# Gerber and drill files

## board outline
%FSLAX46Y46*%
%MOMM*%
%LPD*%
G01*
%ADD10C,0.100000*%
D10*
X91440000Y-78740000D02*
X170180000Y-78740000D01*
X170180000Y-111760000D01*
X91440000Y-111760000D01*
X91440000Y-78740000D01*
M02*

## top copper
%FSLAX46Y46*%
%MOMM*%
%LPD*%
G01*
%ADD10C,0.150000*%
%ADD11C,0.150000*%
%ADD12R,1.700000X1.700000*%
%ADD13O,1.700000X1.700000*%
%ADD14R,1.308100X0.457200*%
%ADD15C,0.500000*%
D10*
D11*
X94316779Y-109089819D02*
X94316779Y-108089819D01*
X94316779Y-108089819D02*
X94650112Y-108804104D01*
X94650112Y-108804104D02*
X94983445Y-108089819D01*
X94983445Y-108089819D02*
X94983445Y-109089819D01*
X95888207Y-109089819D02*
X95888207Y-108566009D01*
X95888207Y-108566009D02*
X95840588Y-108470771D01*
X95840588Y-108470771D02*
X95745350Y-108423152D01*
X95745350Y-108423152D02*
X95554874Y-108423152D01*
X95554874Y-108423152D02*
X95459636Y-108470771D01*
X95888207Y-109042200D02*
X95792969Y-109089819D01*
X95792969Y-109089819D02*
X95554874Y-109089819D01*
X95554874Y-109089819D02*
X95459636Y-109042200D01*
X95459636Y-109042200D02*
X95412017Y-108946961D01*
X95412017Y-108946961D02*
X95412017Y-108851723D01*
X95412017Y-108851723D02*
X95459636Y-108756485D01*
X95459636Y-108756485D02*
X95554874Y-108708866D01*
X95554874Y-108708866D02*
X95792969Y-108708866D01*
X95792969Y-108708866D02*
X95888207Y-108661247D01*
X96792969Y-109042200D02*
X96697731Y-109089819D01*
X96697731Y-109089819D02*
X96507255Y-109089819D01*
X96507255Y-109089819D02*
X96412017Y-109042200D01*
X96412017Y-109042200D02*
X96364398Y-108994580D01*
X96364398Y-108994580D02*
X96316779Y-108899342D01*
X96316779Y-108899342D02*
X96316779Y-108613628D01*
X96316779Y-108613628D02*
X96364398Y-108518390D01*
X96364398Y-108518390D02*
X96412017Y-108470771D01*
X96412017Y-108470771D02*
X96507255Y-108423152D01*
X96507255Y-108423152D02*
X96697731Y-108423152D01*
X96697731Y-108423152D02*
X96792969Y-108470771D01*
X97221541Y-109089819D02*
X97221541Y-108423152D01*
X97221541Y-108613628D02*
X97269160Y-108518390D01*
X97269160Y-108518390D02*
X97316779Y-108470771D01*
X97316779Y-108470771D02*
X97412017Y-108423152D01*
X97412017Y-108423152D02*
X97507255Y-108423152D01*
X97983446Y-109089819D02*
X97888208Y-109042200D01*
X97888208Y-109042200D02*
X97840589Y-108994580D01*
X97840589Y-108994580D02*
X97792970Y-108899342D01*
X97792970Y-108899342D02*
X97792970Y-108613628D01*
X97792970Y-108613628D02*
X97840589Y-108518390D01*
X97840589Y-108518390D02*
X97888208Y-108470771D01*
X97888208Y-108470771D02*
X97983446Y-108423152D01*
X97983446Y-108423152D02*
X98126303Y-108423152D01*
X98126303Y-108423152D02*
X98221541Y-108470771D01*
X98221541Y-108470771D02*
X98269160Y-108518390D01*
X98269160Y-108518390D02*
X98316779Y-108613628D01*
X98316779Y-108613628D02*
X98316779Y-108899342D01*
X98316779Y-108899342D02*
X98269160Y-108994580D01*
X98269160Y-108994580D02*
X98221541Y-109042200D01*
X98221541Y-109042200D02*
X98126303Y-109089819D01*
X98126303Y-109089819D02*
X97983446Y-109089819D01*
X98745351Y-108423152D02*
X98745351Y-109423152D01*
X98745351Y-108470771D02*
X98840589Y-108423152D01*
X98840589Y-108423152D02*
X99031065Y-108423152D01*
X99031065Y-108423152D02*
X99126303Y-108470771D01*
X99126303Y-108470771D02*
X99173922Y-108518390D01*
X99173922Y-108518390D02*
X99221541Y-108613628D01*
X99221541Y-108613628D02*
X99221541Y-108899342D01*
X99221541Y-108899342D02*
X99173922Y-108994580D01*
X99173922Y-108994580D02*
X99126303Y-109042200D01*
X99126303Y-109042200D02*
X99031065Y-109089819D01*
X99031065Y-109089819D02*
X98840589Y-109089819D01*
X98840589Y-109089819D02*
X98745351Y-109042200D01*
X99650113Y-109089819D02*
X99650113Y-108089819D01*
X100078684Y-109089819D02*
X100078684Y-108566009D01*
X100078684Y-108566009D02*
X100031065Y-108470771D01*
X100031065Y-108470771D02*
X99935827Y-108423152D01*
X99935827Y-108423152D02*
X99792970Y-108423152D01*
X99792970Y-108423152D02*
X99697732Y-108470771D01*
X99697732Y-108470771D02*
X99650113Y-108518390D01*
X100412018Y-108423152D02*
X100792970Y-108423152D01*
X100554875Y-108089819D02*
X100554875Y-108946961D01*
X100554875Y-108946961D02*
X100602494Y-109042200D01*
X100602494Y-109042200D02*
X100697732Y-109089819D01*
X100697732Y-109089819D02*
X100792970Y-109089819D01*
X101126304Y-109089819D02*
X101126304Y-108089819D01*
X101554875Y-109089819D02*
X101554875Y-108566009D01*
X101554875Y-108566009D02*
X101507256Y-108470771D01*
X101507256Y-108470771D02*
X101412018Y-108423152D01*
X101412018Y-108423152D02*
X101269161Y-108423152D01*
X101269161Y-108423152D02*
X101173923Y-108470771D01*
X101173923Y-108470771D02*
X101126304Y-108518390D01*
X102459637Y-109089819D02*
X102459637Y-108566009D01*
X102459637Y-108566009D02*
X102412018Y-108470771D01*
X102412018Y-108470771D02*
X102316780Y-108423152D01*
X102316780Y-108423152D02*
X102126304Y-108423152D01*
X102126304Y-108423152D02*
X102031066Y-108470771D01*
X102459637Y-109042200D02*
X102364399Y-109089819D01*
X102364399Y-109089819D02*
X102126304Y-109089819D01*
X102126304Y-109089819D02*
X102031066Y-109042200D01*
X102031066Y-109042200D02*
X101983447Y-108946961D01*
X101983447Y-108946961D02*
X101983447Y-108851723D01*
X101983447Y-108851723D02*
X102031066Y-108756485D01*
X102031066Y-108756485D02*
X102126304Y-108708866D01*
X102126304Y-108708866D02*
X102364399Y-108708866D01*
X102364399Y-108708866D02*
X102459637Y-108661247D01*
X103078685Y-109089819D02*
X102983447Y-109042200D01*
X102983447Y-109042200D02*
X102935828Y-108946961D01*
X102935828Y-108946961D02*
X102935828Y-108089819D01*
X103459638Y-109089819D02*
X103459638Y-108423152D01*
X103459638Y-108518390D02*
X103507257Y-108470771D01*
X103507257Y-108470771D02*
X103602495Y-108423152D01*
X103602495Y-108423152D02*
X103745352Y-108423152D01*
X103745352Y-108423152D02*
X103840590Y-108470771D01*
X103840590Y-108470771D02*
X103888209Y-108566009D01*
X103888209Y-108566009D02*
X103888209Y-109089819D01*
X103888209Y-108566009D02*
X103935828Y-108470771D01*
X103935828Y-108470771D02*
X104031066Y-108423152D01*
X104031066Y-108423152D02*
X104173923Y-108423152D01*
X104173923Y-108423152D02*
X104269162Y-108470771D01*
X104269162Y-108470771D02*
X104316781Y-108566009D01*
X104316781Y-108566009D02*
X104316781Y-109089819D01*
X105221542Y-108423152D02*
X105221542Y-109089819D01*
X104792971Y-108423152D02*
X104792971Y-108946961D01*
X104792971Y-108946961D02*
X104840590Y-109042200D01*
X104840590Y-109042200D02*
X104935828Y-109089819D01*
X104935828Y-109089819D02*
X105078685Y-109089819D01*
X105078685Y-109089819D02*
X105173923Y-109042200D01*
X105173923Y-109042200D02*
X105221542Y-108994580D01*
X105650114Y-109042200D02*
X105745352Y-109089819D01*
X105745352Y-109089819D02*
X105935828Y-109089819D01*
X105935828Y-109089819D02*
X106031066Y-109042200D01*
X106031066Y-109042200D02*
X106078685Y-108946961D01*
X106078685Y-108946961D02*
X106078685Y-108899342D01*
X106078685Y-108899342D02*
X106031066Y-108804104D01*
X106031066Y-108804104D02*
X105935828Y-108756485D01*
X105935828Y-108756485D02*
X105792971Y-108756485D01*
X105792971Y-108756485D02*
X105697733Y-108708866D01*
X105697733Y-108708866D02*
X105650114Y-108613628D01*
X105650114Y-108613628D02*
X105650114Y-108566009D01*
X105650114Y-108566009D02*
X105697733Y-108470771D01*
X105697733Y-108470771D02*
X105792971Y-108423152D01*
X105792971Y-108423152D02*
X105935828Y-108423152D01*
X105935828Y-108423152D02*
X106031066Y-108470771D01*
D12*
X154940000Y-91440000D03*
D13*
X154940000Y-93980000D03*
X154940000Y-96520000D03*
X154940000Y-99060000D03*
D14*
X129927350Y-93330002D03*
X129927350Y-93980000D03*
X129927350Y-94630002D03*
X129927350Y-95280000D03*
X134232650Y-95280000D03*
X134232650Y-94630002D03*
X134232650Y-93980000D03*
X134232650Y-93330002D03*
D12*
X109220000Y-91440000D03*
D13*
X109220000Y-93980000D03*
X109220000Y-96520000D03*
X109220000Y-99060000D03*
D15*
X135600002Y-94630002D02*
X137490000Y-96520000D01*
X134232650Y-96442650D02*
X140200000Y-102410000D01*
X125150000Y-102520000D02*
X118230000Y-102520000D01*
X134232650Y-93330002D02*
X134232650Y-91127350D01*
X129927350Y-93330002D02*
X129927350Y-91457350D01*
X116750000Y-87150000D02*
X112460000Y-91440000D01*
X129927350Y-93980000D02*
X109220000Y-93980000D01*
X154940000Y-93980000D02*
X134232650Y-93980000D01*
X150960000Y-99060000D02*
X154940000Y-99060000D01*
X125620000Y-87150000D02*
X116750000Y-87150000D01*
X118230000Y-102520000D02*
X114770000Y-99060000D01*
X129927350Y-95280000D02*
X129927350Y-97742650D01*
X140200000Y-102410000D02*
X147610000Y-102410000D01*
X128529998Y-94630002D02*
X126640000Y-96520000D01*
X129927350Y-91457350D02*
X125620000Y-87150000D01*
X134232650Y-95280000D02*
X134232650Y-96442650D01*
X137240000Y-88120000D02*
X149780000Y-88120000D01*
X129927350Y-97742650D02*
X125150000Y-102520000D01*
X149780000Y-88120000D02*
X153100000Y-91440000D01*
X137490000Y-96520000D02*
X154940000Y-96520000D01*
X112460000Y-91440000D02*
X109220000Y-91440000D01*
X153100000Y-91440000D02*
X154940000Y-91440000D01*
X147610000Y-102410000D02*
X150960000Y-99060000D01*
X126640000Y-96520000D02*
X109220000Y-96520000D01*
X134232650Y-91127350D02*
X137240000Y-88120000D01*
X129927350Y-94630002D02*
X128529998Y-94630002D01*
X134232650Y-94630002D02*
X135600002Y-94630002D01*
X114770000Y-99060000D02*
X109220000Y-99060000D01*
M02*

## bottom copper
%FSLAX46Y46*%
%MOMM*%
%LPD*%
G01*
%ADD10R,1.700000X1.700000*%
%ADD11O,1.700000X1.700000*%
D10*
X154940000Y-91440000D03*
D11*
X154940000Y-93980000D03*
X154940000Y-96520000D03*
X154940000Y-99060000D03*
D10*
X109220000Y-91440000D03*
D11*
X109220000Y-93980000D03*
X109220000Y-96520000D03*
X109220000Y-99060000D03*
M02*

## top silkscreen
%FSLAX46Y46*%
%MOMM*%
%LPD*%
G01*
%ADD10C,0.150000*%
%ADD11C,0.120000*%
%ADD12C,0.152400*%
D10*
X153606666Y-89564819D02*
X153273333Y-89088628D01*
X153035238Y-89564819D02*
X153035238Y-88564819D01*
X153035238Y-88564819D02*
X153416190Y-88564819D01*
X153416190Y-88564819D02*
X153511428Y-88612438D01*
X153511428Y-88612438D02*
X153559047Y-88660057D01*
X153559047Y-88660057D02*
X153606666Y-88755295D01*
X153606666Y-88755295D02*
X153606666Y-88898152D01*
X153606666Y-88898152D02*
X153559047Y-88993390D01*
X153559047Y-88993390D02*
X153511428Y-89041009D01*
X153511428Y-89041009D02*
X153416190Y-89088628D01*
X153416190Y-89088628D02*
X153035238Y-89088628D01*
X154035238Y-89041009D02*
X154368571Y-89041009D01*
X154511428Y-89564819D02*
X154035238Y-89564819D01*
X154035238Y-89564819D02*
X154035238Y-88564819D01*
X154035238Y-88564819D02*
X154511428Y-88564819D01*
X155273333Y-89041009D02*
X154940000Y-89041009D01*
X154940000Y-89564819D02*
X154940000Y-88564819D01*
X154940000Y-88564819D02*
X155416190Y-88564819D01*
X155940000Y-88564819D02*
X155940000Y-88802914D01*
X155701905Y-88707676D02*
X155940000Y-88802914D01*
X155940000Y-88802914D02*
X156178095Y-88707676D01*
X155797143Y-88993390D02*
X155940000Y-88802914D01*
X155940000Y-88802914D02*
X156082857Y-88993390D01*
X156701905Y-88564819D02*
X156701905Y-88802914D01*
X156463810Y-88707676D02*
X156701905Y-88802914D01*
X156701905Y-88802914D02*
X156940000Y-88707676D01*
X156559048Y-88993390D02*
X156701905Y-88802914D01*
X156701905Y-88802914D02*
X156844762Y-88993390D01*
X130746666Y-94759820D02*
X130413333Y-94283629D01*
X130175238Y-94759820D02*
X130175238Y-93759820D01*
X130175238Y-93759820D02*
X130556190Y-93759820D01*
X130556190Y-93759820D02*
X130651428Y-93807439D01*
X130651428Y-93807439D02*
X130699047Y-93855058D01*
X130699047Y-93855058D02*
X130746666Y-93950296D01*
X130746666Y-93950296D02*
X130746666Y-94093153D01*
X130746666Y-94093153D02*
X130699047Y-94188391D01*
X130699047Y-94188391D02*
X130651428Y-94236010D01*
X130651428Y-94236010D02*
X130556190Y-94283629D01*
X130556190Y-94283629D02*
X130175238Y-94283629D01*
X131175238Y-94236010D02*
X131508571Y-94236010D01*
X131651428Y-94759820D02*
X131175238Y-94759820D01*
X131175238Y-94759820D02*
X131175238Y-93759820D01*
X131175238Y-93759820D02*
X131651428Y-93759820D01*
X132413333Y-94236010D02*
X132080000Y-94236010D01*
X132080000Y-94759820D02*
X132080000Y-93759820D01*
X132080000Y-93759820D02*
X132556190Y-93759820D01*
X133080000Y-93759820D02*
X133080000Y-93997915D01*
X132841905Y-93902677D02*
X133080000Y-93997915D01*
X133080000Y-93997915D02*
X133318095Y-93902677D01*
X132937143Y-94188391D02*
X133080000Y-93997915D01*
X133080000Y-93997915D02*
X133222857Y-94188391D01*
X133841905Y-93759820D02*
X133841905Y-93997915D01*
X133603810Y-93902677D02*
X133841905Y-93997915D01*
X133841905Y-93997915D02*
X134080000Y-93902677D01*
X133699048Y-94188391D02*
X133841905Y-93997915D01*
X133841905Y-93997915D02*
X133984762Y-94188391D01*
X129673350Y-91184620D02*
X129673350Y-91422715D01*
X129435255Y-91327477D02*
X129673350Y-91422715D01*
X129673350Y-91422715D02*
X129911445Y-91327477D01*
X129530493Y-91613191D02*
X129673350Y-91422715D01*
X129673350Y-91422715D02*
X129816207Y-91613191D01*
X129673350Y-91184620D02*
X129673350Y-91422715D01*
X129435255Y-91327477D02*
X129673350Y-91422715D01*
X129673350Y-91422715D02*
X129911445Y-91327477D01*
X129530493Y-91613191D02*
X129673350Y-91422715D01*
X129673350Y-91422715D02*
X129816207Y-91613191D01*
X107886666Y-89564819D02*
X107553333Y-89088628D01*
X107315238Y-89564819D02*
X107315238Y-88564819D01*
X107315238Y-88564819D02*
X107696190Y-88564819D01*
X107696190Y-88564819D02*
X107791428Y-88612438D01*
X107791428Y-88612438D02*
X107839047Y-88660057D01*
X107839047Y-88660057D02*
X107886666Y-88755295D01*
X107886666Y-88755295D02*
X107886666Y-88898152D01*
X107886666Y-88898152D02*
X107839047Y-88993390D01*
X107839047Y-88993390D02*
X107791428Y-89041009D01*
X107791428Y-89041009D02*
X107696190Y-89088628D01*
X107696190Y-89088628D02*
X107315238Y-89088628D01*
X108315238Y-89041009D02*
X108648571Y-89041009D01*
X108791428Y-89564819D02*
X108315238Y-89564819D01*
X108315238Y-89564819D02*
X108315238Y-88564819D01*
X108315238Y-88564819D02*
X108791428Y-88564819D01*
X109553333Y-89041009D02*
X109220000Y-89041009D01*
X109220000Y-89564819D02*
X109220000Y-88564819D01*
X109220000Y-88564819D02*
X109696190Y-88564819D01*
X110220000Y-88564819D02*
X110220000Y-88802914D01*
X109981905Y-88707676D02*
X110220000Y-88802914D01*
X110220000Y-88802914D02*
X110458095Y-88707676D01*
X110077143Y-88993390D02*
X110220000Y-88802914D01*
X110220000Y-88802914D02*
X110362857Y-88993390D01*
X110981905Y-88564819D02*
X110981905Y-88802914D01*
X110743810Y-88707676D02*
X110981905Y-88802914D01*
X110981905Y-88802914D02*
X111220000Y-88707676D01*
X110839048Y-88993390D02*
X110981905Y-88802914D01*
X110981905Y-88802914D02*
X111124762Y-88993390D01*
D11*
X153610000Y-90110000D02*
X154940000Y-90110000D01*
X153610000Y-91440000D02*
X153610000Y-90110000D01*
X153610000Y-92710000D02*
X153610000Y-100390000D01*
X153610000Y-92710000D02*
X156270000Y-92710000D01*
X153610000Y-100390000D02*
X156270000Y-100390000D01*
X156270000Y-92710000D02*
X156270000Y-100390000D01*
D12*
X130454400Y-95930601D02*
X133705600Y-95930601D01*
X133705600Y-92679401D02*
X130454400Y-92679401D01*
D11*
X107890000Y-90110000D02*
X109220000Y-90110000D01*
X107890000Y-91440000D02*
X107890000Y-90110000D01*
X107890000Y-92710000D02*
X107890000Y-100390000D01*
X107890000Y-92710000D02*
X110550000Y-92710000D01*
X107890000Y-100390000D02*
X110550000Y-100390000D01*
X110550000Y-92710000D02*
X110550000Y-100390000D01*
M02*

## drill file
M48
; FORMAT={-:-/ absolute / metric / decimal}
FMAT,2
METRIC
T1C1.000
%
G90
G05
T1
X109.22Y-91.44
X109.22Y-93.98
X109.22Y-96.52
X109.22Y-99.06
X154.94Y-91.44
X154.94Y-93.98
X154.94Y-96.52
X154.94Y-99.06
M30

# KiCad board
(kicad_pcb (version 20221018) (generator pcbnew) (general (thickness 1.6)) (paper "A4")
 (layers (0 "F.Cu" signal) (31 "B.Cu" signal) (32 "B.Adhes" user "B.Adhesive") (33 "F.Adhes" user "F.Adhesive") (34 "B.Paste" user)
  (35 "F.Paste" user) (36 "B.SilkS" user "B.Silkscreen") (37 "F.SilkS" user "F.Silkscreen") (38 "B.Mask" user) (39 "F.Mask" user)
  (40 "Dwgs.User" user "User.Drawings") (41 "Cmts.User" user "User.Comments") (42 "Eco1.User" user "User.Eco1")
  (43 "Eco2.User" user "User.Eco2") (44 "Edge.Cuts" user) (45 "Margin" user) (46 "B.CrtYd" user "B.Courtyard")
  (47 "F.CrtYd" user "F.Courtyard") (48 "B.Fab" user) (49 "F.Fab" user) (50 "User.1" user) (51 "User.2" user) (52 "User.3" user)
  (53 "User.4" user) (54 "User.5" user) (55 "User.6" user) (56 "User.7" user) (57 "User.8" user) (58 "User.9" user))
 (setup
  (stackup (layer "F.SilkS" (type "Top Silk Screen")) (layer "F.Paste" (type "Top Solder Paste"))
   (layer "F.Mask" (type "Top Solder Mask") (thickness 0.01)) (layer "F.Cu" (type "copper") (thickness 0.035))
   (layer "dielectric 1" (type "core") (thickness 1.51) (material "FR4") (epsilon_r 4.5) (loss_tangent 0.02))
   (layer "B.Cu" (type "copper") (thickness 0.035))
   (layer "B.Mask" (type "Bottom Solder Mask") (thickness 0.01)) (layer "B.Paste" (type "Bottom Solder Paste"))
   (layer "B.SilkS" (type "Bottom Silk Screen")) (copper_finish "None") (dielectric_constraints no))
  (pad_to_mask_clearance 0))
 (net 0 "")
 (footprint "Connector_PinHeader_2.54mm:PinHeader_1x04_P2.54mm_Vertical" (layer "F.Cu") (at 154.94 91.44)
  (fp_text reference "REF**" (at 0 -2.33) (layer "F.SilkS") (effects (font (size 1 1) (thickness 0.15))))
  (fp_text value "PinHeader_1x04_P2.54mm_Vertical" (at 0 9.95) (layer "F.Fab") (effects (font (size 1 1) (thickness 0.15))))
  (fp_line (start -1.33 -1.33) (end 0 -1.33) (stroke (width 0.12) (type solid)) (layer "F.SilkS"))
  (fp_line (start -1.33 0) (end -1.33 -1.33) (stroke (width 0.12) (type solid)) (layer "F.SilkS"))
  (fp_line (start -1.33 1.27) (end -1.33 8.95) (stroke (width 0.12) (type solid)) (layer "F.SilkS"))
  (fp_line (start -1.33 1.27) (end 1.33 1.27) (stroke (width 0.12) (type solid)) (layer "F.SilkS"))
  (fp_line (start -1.33 8.95) (end 1.33 8.95) (stroke (width 0.12) (type solid)) (layer "F.SilkS"))
  (fp_line (start 1.33 1.27) (end 1.33 8.95) (stroke (width 0.12) (type solid)) (layer "F.SilkS"))
  (pad "1" thru_hole rect (at 0 0) (size 1.7 1.7) (drill 1) (layers "*.Cu" "*.Mask"))
  (pad "2" thru_hole oval (at 0 2.54) (size 1.7 1.7) (drill 1) (layers "*.Cu" "*.Mask"))
  (pad "3" thru_hole oval (at 0 5.08) (size 1.7 1.7) (drill 1) (layers "*.Cu" "*.Mask"))
  (pad "4" thru_hole oval (at 0 7.62) (size 1.7 1.7) (drill 1) (layers "*.Cu" "*.Mask")))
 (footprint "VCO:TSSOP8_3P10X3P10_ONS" (layer "F.Cu") (at 132.08 94.305001)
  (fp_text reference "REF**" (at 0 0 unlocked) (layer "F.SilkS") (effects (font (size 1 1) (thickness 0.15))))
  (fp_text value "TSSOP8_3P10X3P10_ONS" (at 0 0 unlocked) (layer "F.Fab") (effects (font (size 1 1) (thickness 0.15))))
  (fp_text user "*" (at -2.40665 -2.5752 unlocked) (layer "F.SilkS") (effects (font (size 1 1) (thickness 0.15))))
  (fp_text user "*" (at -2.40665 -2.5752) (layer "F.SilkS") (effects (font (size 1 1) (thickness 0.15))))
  (fp_line (start -1.6256 1.6256) (end 1.6256 1.6256) (stroke (width 0.1524) (type solid)) (layer "F.SilkS"))
  (fp_line (start 1.6256 -1.6256) (end -1.6256 -1.6256) (stroke (width 0.1524) (type solid)) (layer "F.SilkS"))
  (pad "1" smd rect (at -2.15265 -0.974999) (size 1.3081 0.4572) (layers "F.Cu" "F.Paste" "F.Mask"))
  (pad "2" smd rect (at -2.15265 -0.325001) (size 1.3081 0.4572) (layers "F.Cu" "F.Paste" "F.Mask"))
  (pad "3" smd rect (at -2.15265 0.325001) (size 1.3081 0.4572) (layers "F.Cu" "F.Paste" "F.Mask"))
  (pad "4" smd rect (at -2.15265 0.974999) (size 1.3081 0.4572) (layers "F.Cu" "F.Paste" "F.Mask"))
  (pad "5" smd rect (at 2.15265 0.974999) (size 1.3081 0.4572) (layers "F.Cu" "F.Paste" "F.Mask"))
  (pad "6" smd rect (at 2.15265 0.325001) (size 1.3081 0.4572) (layers "F.Cu" "F.Paste" "F.Mask"))
  (pad "7" smd rect (at 2.15265 -0.325001) (size 1.3081 0.4572) (layers "F.Cu" "F.Paste" "F.Mask"))
  (pad "8" smd rect (at 2.15265 -0.974999) (size 1.3081 0.4572) (layers "F.Cu" "F.Paste" "F.Mask")))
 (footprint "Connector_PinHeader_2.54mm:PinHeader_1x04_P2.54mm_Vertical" (layer "F.Cu") (at 109.22 91.44)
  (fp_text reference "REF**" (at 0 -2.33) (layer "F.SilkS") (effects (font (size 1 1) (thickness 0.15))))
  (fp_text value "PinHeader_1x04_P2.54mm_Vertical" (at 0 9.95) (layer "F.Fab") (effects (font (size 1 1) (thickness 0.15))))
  (fp_line (start -1.33 -1.33) (end 0 -1.33) (stroke (width 0.12) (type solid)) (layer "F.SilkS"))
  (fp_line (start -1.33 0) (end -1.33 -1.33) (stroke (width 0.12) (type solid)) (layer "F.SilkS"))
  (fp_line (start -1.33 1.27) (end -1.33 8.95) (stroke (width 0.12) (type solid)) (layer "F.SilkS"))
  (fp_line (start -1.33 1.27) (end 1.33 1.27) (stroke (width 0.12) (type solid)) (layer "F.SilkS"))
  (fp_line (start -1.33 8.95) (end 1.33 8.95) (stroke (width 0.12) (type solid)) (layer "F.SilkS"))
  (fp_line (start 1.33 1.27) (end 1.33 8.95) (stroke (width 0.12) (type solid)) (layer "F.SilkS"))
  (pad "1" thru_hole rect (at 0 0) (size 1.7 1.7) (drill 1) (layers "*.Cu" "*.Mask"))
  (pad "2" thru_hole oval (at 0 2.54) (size 1.7 1.7) (drill 1) (layers "*.Cu" "*.Mask"))
  (pad "3" thru_hole oval (at 0 5.08) (size 1.7 1.7) (drill 1) (layers "*.Cu" "*.Mask"))
  (pad "4" thru_hole oval (at 0 7.62) (size 1.7 1.7) (drill 1) (layers "*.Cu" "*.Mask")))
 (gr_rect (start 91.44 78.74) (end 170.18 111.76) (stroke (width 0.1) (type default)) (fill none) (layer "Edge.Cuts"))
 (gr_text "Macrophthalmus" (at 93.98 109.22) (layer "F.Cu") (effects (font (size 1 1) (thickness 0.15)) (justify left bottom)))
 (segment (start 135.600002 94.630002) (end 137.49 96.52) (width 0.5) (layer "F.Cu") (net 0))
 (segment (start 134.23265 96.44265) (end 140.2 102.41) (width 0.5) (layer "F.Cu") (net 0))
 (segment (start 125.15 102.52) (end 118.23 102.52) (width 0.5) (layer "F.Cu") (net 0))
 (segment (start 134.23265 93.330002) (end 134.23265 91.12735) (width 0.5) (layer "F.Cu") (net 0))
 (segment (start 129.92735 93.330002) (end 129.92735 91.45735) (width 0.5) (layer "F.Cu") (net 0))
 (segment (start 116.75 87.15) (end 112.46 91.44) (width 0.5) (layer "F.Cu") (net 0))
 (segment (start 129.92735 93.98) (end 109.22 93.98) (width 0.5) (layer "F.Cu") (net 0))
 (segment (start 154.94 93.98) (end 134.23265 93.98) (width 0.5) (layer "F.Cu") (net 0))
 (segment (start 150.96 99.06) (end 154.94 99.06) (width 0.5) (layer "F.Cu") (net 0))
 (segment (start 125.62 87.15) (end 116.75 87.15) (width 0.5) (layer "F.Cu") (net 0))
 (segment (start 118.23 102.52) (end 114.77 99.06) (width 0.5) (layer "F.Cu") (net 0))
 (segment (start 129.92735 95.28) (end 129.92735 97.74265) (width 0.5) (layer "F.Cu") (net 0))
 (segment (start 140.2 102.41) (end 147.61 102.41) (width 0.5) (layer "F.Cu") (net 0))
 (segment (start 128.529998 94.630002) (end 126.64 96.52) (width 0.5) (layer "F.Cu") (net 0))
 (segment (start 129.92735 91.45735) (end 125.62 87.15) (width 0.5) (layer "F.Cu") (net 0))
 (segment (start 134.23265 95.28) (end 134.23265 96.44265) (width 0.5) (layer "F.Cu") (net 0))
 (segment (start 137.24 88.12) (end 149.78 88.12) (width 0.5) (layer "F.Cu") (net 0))
 (segment (start 129.92735 97.74265) (end 125.15 102.52) (width 0.5) (layer "F.Cu") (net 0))
 (segment (start 149.78 88.12) (end 153.1 91.44) (width 0.5) (layer "F.Cu") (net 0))
 (segment (start 137.49 96.52) (end 154.94 96.52) (width 0.5) (layer "F.Cu") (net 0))
 (segment (start 112.46 91.44) (end 109.22 91.44) (width 0.5) (layer "F.Cu") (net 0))
 (segment (start 153.1 91.44) (end 154.94 91.44) (width 0.5) (layer "F.Cu") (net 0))
 (segment (start 147.61 102.41) (end 150.96 99.06) (width 0.5) (layer "F.Cu") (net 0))
 (segment (start 126.64 96.52) (end 109.22 96.52) (width 0.5) (layer "F.Cu") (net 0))
 (segment (start 134.23265 91.12735) (end 137.24 88.12) (width 0.5) (layer "F.Cu") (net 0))
 (segment (start 129.92735 94.630002) (end 128.529998 94.630002) (width 0.5) (layer "F.Cu") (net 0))
 (segment (start 134.23265 94.630002) (end 135.600002 94.630002) (width 0.5) (layer "F.Cu") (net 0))
 (segment (start 114.77 99.06) (end 109.22 99.06) (width 0.5) (layer "F.Cu") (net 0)))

